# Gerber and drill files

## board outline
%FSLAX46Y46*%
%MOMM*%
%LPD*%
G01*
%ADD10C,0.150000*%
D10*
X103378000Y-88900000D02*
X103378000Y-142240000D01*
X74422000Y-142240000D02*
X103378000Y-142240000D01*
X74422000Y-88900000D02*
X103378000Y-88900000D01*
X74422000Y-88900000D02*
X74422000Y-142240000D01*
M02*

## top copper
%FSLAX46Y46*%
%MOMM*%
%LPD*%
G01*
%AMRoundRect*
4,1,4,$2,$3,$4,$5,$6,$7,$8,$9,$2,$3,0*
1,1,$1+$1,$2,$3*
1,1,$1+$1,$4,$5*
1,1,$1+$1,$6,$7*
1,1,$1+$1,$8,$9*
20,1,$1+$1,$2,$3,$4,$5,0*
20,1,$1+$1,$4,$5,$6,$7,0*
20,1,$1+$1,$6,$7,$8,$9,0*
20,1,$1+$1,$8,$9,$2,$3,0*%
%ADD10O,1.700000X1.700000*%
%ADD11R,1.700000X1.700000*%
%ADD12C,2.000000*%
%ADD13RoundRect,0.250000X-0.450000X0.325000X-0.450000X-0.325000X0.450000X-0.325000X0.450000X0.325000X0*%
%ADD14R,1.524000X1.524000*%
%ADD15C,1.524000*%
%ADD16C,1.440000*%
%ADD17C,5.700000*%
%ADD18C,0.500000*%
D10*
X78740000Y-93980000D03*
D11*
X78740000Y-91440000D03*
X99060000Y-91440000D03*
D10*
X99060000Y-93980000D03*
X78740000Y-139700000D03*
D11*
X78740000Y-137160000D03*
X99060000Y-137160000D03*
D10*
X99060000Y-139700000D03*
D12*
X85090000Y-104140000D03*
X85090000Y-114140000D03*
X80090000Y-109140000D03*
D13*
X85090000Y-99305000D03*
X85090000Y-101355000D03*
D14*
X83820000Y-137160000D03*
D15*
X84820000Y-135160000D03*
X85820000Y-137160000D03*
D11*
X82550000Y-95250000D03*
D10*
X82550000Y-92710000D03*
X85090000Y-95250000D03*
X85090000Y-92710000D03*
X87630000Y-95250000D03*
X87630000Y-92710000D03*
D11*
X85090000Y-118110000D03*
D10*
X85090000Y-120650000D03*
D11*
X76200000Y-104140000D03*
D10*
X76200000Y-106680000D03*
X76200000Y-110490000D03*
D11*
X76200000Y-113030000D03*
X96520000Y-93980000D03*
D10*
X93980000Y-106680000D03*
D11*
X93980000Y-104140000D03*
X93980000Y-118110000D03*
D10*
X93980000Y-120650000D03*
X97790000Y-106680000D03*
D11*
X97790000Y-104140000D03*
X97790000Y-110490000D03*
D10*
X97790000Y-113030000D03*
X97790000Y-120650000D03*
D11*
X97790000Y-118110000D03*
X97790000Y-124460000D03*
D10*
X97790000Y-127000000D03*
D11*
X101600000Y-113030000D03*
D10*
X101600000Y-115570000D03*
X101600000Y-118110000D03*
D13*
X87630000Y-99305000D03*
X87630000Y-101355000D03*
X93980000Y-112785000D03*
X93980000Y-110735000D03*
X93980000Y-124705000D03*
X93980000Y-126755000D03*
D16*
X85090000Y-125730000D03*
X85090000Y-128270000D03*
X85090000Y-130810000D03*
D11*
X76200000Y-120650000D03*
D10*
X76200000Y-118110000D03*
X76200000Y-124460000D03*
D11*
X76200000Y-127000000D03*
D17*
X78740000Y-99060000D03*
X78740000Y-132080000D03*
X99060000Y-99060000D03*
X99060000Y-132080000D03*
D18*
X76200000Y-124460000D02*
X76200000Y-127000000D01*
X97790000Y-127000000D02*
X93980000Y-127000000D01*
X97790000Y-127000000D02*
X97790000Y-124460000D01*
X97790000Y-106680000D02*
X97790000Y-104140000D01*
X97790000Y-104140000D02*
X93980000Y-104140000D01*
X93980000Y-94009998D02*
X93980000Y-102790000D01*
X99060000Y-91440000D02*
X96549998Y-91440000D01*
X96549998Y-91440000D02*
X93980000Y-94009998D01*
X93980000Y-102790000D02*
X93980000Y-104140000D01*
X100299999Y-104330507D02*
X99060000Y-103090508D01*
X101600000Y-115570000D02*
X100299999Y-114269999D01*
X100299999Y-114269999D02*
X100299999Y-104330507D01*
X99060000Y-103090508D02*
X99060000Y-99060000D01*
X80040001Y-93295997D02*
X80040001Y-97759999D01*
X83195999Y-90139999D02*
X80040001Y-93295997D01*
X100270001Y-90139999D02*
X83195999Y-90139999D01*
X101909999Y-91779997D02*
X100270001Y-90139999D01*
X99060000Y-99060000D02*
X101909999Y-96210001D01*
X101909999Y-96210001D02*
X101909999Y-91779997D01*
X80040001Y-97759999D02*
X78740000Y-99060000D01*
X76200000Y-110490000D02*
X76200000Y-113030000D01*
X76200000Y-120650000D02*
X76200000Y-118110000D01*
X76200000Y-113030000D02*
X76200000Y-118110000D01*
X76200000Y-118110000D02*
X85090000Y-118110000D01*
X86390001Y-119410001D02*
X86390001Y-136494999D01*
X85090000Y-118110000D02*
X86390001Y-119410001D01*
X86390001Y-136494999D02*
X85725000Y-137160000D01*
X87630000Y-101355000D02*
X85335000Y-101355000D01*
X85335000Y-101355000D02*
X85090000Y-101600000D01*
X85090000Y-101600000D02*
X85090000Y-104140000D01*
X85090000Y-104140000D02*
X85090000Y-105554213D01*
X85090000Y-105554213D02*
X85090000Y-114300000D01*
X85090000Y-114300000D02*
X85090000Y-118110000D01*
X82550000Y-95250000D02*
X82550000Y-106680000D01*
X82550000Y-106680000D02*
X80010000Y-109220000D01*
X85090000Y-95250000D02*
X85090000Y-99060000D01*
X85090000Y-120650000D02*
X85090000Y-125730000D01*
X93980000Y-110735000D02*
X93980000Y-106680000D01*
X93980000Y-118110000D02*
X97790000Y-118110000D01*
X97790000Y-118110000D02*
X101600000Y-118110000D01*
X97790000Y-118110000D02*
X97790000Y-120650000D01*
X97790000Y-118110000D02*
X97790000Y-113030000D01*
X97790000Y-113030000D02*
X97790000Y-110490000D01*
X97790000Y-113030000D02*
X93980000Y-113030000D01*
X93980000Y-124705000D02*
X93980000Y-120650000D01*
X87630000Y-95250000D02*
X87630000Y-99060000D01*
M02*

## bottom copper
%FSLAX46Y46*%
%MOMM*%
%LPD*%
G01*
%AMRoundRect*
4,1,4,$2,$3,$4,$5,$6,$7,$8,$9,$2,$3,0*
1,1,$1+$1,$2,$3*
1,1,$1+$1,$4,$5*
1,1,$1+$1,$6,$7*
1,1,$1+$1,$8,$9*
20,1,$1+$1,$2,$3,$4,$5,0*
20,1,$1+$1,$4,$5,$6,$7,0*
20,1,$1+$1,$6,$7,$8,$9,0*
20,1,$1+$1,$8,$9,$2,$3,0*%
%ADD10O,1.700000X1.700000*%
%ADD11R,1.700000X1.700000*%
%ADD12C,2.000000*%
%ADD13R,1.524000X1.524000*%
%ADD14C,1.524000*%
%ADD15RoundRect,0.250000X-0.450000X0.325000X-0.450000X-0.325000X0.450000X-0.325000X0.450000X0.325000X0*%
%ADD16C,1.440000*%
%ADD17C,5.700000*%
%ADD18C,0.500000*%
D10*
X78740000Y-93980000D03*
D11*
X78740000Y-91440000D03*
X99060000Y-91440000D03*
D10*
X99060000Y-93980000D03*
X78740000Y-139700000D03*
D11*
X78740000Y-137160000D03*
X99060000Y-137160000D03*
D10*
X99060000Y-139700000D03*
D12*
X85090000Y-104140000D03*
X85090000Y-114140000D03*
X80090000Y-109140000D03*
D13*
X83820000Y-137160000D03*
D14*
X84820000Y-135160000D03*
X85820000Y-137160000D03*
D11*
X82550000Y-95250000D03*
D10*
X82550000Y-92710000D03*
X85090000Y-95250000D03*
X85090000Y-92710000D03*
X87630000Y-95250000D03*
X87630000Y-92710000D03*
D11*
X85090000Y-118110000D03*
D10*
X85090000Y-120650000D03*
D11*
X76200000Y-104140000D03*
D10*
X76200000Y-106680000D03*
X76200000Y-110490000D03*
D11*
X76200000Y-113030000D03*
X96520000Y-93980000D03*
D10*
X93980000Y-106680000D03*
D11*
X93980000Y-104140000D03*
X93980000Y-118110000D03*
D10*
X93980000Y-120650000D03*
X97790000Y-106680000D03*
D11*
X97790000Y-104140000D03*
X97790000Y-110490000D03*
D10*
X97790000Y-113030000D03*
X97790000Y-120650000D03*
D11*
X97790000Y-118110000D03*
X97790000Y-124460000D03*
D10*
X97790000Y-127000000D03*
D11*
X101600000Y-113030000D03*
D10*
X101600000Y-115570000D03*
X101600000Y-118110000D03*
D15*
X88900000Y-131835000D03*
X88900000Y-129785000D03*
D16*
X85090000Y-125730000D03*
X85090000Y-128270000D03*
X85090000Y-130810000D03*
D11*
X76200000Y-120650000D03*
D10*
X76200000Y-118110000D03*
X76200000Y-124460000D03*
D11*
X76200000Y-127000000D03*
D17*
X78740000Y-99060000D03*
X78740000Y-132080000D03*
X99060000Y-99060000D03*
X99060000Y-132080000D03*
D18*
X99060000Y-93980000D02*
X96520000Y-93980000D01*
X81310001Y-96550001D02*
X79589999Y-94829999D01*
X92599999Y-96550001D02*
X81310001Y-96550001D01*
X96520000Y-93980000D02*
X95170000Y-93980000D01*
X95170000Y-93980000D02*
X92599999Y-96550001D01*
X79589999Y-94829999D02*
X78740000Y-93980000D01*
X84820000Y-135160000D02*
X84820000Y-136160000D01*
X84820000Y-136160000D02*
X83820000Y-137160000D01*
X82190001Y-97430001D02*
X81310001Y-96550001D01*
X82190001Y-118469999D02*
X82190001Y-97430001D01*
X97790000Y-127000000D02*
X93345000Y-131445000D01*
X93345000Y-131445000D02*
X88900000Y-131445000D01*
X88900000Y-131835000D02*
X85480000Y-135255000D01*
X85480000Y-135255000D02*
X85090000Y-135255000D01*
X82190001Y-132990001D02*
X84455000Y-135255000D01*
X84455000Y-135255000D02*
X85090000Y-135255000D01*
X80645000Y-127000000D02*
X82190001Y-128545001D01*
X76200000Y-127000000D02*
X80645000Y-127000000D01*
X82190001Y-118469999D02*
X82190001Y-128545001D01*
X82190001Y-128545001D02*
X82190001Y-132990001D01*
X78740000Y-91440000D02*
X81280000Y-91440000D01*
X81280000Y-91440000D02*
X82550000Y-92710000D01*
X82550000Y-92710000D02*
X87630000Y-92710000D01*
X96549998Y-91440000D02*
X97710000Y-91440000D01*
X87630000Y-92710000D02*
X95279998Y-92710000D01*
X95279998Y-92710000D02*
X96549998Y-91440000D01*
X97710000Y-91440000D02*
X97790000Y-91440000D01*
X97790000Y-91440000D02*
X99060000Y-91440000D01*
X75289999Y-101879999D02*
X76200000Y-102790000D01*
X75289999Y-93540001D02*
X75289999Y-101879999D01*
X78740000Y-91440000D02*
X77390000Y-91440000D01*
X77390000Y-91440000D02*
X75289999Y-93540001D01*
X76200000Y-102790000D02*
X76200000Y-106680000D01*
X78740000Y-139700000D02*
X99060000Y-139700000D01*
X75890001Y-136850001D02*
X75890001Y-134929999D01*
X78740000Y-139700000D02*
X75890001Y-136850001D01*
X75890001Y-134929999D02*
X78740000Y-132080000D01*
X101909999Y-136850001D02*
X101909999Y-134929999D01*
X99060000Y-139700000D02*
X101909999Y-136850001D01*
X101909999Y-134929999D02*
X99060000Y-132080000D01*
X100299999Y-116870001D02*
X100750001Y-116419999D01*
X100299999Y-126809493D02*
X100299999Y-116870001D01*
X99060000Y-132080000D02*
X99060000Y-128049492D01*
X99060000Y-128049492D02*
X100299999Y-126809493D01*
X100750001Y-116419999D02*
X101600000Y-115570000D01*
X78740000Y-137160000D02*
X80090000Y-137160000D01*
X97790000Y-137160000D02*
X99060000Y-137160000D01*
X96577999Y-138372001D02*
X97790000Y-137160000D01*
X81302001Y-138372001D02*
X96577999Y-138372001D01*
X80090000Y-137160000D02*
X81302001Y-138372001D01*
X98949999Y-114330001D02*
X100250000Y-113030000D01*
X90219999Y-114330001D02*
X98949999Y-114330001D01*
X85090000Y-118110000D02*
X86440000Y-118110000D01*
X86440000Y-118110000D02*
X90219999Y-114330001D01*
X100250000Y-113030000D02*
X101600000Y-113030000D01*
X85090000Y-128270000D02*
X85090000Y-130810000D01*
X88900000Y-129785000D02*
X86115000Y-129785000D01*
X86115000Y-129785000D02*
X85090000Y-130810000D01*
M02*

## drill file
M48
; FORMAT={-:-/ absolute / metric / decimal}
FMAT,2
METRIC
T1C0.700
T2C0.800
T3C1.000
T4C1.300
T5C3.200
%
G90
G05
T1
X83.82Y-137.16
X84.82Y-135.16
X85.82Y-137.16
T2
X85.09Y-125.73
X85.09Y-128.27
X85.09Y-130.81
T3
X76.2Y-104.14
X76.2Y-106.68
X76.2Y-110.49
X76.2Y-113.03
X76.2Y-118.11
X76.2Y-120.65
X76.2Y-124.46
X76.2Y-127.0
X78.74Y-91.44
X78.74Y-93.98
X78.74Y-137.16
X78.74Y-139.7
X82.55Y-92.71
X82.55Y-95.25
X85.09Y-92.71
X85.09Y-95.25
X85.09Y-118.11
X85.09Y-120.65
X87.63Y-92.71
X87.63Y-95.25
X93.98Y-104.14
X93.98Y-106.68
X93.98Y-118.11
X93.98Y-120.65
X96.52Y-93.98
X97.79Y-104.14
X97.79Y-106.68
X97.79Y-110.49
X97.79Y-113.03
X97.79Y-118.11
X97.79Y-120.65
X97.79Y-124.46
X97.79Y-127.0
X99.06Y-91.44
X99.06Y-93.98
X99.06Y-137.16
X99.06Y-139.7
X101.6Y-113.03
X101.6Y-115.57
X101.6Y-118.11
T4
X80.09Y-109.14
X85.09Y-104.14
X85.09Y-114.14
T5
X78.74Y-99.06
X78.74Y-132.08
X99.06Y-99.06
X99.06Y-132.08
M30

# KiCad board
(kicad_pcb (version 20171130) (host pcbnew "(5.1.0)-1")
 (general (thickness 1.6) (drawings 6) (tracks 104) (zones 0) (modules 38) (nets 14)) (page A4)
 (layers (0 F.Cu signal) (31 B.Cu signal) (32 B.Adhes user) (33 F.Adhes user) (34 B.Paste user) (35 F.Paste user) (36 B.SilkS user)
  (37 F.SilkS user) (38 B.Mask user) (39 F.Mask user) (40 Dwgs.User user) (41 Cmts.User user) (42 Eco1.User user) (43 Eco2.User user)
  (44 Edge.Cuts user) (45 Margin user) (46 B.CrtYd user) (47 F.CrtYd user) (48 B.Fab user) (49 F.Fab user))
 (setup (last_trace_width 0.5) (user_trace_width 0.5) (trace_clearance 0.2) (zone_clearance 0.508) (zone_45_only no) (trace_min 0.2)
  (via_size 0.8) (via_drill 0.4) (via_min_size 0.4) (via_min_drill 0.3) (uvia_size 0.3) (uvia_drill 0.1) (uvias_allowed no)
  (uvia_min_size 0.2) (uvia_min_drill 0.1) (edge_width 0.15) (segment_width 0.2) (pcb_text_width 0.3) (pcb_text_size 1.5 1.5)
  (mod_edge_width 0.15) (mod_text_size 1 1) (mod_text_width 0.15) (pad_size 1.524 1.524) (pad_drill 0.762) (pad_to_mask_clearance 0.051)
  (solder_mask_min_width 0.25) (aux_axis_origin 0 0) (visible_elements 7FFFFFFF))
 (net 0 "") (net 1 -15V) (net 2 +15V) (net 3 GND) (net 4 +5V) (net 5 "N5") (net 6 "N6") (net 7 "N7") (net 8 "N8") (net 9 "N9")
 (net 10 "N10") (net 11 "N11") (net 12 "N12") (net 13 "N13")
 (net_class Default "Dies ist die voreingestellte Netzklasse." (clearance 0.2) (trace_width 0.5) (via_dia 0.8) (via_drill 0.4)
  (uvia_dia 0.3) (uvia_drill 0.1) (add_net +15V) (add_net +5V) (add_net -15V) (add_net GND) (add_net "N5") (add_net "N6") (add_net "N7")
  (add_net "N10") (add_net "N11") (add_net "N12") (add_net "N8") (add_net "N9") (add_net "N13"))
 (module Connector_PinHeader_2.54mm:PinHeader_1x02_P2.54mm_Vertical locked (layer B.Cu) (at 78.74 91.44 180)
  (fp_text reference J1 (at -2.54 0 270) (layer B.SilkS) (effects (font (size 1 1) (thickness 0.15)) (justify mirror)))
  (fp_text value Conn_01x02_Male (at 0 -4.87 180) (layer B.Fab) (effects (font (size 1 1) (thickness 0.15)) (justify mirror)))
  (pad 2 thru_hole oval (at 0 -2.54 180) (size 1.7 1.7) (drill 1) (layers *.Cu *.Mask) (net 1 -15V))
  (pad 1 thru_hole rect (at 0 0 180) (size 1.7 1.7) (drill 1) (layers *.Cu *.Mask) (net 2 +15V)))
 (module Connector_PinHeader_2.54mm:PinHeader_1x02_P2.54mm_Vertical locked (layer B.Cu) (at 99.06 91.44 180)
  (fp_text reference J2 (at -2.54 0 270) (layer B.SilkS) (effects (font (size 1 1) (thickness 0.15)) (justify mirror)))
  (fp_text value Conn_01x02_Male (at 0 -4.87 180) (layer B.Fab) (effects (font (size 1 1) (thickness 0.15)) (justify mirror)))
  (pad 1 thru_hole rect (at 0 0 180) (size 1.7 1.7) (drill 1) (layers *.Cu *.Mask) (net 2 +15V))
  (pad 2 thru_hole oval (at 0 -2.54 180) (size 1.7 1.7) (drill 1) (layers *.Cu *.Mask) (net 1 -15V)))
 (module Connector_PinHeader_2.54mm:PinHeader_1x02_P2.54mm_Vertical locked (layer B.Cu) (at 78.74 137.16 180)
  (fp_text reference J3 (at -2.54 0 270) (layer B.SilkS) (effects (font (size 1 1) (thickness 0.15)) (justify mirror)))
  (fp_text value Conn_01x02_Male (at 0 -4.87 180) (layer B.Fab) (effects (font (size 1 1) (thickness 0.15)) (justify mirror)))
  (pad 2 thru_hole oval (at 0 -2.54 180) (size 1.7 1.7) (drill 1) (layers *.Cu *.Mask) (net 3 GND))
  (pad 1 thru_hole rect (at 0 0 180) (size 1.7 1.7) (drill 1) (layers *.Cu *.Mask) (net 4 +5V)))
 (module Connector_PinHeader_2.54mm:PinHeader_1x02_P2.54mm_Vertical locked (layer B.Cu) (at 99.06 137.16 180)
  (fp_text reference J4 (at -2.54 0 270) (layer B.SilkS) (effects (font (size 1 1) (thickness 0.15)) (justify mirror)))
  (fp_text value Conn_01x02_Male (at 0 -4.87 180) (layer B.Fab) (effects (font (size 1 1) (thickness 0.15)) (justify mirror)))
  (pad 1 thru_hole rect (at 0 0 180) (size 1.7 1.7) (drill 1) (layers *.Cu *.Mask) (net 4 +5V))
  (pad 2 thru_hole oval (at 0 -2.54 180) (size 1.7 1.7) (drill 1) (layers *.Cu *.Mask) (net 3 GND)))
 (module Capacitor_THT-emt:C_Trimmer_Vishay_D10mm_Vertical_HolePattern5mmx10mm (layer F.Cu) (at 85.09 104.14 270)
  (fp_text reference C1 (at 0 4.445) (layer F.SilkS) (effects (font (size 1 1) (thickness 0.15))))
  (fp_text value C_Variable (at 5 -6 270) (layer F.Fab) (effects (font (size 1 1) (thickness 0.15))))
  (pad 1 thru_hole circle (at 0 0 270) (size 2 2) (drill 1.3) (layers *.Cu *.Mask) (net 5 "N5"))
  (pad 1 thru_hole circle (at 10 0 270) (size 2 2) (drill 1.3) (layers *.Cu *.Mask) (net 5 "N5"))
  (pad 2 thru_hole circle (at 5 5 270) (size 2 2) (drill 1.3) (layers *.Cu *.Mask) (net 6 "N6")))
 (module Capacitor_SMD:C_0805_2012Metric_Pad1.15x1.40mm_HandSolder (layer F.Cu) (at 85.09 100.33 270)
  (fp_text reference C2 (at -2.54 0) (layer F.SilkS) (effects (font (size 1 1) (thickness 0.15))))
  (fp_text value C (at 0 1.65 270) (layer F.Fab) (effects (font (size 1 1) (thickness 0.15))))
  (pad 1 smd roundrect (at -1.025 0 270) (size 1.15 1.4) (layers F.Cu F.Paste F.Mask) (roundrect_rratio 0.217391) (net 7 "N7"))
  (pad 2 smd roundrect (at 1.025 0 270) (size 1.15 1.4) (layers F.Cu F.Paste F.Mask) (roundrect_rratio 0.217391) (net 5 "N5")))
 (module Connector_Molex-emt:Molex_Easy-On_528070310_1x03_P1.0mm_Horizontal (layer F.Cu) (at 83.82 137.16)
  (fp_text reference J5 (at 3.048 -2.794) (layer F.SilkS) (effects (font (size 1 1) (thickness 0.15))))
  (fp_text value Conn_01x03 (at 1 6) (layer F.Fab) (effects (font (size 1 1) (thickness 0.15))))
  (pad 1 thru_hole rect (at 0 0) (size 1.524 1.524) (drill 0.7) (layers *.Cu *.Mask) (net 1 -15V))
  (pad 2 thru_hole circle (at 1 -2) (size 1.524 1.524) (drill 0.7) (layers *.Cu *.Mask) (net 1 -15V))
  (pad 3 thru_hole circle (at 2 0) (size 1.524 1.524) (drill 0.7) (layers *.Cu *.Mask) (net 5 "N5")))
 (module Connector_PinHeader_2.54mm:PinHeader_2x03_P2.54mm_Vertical (layer F.Cu) (at 82.55 95.25 90)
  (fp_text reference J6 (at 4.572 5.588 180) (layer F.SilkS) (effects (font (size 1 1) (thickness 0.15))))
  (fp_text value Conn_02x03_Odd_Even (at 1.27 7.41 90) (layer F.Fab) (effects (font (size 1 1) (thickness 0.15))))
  (pad 1 thru_hole rect (at 0 0 90) (size 1.7 1.7) (drill 1) (layers *.Cu *.Mask) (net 6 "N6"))
  (pad 2 thru_hole oval (at 2.54 0 90) (size 1.7 1.7) (drill 1) (layers *.Cu *.Mask) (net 2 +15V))
  (pad 3 thru_hole oval (at 0 2.54 90) (size 1.7 1.7) (drill 1) (layers *.Cu *.Mask) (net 7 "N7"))
  (pad 4 thru_hole oval (at 2.54 2.54 90) (size 1.7 1.7) (drill 1) (layers *.Cu *.Mask) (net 2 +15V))
  (pad 5 thru_hole oval (at 0 5.08 90) (size 1.7 1.7) (drill 1) (layers *.Cu *.Mask) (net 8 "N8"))
  (pad 6 thru_hole oval (at 2.54 5.08 90) (size 1.7 1.7) (drill 1) (layers *.Cu *.Mask) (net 2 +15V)))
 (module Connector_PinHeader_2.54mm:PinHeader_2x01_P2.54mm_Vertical (layer F.Cu) (at 85.09 118.11 270)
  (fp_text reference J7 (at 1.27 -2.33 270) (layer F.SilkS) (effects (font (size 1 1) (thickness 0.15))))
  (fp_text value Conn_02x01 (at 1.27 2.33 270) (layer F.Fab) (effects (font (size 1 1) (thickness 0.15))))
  (pad 1 thru_hole rect (at 0 0 270) (size 1.7 1.7) (drill 1) (layers *.Cu *.Mask) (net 5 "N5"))
  (pad 2 thru_hole oval (at 2.54 0 270) (size 1.7 1.7) (drill 1) (layers *.Cu *.Mask) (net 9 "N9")))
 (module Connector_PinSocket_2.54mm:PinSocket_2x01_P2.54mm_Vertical (layer F.Cu) (at 76.2 104.14 90)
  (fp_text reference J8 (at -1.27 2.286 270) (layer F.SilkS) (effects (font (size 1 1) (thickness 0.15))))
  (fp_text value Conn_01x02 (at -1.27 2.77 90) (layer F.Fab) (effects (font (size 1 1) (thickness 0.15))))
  (pad 1 thru_hole rect (at 0 0 90) (size 1.7 1.7) (drill 1) (layers *.Cu *.Mask) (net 2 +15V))
  (pad 2 thru_hole oval (at -2.54 0 90) (size 1.7 1.7) (drill 1) (layers *.Cu *.Mask) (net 2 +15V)))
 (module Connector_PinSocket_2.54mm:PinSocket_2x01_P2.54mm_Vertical (layer F.Cu) (at 76.2 113.03 270)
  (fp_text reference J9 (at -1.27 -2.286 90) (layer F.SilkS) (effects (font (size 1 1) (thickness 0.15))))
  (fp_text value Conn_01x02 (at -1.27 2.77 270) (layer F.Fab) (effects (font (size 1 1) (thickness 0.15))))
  (pad 2 thru_hole oval (at -2.54 0 270) (size 1.7 1.7) (drill 1) (layers *.Cu *.Mask) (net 5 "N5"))
  (pad 1 thru_hole rect (at 0 0 270) (size 1.7 1.7) (drill 1) (layers *.Cu *.Mask) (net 5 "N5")))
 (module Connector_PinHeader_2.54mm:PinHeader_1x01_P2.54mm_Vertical (layer F.Cu) (at 96.52 93.98)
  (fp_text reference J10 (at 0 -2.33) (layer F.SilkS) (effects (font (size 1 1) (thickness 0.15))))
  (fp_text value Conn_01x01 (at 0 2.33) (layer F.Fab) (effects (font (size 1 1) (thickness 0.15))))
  (pad 1 thru_hole rect (at 0 0) (size 1.7 1.7) (drill 1) (layers *.Cu *.Mask) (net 1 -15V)))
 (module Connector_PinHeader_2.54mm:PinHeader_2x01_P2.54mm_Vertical (layer F.Cu) (at 93.98 104.14 270)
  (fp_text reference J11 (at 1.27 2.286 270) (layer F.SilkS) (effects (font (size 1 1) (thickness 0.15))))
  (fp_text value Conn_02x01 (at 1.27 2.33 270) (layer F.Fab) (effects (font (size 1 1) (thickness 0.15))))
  (pad 2 thru_hole oval (at 2.54 0 270) (size 1.7 1.7) (drill 1) (layers *.Cu *.Mask) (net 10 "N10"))
  (pad 1 thru_hole rect (at 0 0 270) (size 1.7 1.7) (drill 1) (layers *.Cu *.Mask) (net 2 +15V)))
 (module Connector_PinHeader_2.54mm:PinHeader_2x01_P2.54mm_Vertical (layer F.Cu) (at 93.98 118.11 270)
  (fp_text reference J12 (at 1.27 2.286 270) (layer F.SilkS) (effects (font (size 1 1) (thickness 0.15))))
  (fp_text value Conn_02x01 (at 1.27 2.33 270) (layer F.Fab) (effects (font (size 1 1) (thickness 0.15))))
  (pad 1 thru_hole rect (at 0 0 270) (size 1.7 1.7) (drill 1) (layers *.Cu *.Mask) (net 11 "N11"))
  (pad 2 thru_hole oval (at 2.54 0 270) (size 1.7 1.7) (drill 1) (layers *.Cu *.Mask) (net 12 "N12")))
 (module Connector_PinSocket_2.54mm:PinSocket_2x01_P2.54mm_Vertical (layer F.Cu) (at 97.79 104.14 90)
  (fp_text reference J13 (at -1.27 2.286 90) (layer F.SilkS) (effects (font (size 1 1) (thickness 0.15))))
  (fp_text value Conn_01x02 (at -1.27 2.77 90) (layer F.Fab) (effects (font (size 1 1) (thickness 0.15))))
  (pad 2 thru_hole oval (at -2.54 0 90) (size 1.7 1.7) (drill 1) (layers *.Cu *.Mask) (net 2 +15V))
  (pad 1 thru_hole rect (at 0 0 90) (size 1.7 1.7) (drill 1) (layers *.Cu *.Mask) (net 2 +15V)))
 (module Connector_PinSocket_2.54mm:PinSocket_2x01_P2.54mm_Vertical (layer F.Cu) (at 97.79 110.49 90)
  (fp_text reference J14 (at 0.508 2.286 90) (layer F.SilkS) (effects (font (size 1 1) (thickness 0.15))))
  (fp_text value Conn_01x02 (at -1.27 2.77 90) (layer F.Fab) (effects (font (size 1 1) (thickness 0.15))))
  (pad 1 thru_hole rect (at 0 0 90) (size 1.7 1.7) (drill 1) (layers *.Cu *.Mask) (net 11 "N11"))
  (pad 2 thru_hole oval (at -2.54 0 90) (size 1.7 1.7) (drill 1) (layers *.Cu *.Mask) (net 11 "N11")))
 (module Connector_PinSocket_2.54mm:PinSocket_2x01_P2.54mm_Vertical (layer F.Cu) (at 97.79 118.11 90)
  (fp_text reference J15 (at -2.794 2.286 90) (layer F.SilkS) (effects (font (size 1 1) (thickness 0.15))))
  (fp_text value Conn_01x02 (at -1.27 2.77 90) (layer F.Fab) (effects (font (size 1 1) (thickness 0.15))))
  (pad 2 thru_hole oval (at -2.54 0 90) (size 1.7 1.7) (drill 1) (layers *.Cu *.Mask) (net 11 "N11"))
  (pad 1 thru_hole rect (at 0 0 90) (size 1.7 1.7) (drill 1) (layers *.Cu *.Mask) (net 11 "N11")))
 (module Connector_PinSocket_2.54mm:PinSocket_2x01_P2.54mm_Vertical (layer F.Cu) (at 97.79 124.46 90)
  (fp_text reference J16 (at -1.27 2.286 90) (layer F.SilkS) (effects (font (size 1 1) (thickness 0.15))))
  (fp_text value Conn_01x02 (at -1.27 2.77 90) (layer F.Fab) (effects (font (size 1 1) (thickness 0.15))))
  (pad 1 thru_hole rect (at 0 0 90) (size 1.7 1.7) (drill 1) (layers *.Cu *.Mask) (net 1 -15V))
  (pad 2 thru_hole oval (at -2.54 0 90) (size 1.7 1.7) (drill 1) (layers *.Cu *.Mask) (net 1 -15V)))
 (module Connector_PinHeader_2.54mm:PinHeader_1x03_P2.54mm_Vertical (layer F.Cu) (at 101.6 113.03)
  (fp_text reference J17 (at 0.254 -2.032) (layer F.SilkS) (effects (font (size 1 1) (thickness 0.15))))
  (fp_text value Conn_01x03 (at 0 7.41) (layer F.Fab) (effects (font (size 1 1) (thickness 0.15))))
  (pad 1 thru_hole rect (at 0 0) (size 1.7 1.7) (drill 1) (layers *.Cu *.Mask) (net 5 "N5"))
  (pad 2 thru_hole oval (at 0 2.54) (size 1.7 1.7) (drill 1) (layers *.Cu *.Mask) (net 3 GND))
  (pad 3 thru_hole oval (at 0 5.08) (size 1.7 1.7) (drill 1) (layers *.Cu *.Mask) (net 11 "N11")))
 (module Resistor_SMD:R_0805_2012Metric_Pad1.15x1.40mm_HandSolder (layer F.Cu) (at 87.63 100.33 270)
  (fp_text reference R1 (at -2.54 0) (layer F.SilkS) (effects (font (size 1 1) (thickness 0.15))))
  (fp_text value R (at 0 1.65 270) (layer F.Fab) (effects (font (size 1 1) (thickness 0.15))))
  (pad 1 smd roundrect (at -1.025 0 270) (size 1.15 1.4) (layers F.Cu F.Paste F.Mask) (roundrect_rratio 0.217391) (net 8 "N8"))
  (pad 2 smd roundrect (at 1.025 0 270) (size 1.15 1.4) (layers F.Cu F.Paste F.Mask) (roundrect_rratio 0.217391) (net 5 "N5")))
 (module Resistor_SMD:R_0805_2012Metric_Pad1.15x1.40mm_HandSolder (layer B.Cu) (at 88.9 130.81 270)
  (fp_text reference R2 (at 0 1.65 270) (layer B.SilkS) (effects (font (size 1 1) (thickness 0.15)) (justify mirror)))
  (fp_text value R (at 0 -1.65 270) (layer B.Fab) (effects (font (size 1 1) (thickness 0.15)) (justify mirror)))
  (pad 2 smd roundrect (at 1.025 0 270) (size 1.15 1.4) (layers B.Cu B.Paste B.Mask) (roundrect_rratio 0.217391) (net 1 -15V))
  (pad 1 smd roundrect (at -1.025 0 270) (size 1.15 1.4) (layers B.Cu B.Paste B.Mask) (roundrect_rratio 0.217391) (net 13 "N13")))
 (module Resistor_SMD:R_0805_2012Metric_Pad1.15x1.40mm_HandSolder (layer F.Cu) (at 93.98 111.76 270)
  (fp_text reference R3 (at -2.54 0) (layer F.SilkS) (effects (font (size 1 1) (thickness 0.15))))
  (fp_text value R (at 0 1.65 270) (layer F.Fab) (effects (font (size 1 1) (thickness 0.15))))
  (pad 2 smd roundrect (at 1.025 0 270) (size 1.15 1.4) (layers F.Cu F.Paste F.Mask) (roundrect_rratio 0.217391) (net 11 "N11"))
  (pad 1 smd roundrect (at -1.025 0 270) (size 1.15 1.4) (layers F.Cu F.Paste F.Mask) (roundrect_rratio 0.217391) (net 10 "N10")))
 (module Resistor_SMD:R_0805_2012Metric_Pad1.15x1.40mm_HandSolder (layer F.Cu) (at 93.98 125.73 270)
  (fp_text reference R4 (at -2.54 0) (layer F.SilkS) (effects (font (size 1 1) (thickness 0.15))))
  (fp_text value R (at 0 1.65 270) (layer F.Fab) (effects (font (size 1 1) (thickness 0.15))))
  (pad 1 smd roundrect (at -1.025 0 270) (size 1.15 1.4) (layers F.Cu F.Paste F.Mask) (roundrect_rratio 0.217391) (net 12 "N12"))
  (pad 2 smd roundrect (at 1.025 0 270) (size 1.15 1.4) (layers F.Cu F.Paste F.Mask) (roundrect_rratio 0.217391) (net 1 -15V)))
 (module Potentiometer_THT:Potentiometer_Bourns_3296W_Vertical (layer F.Cu) (at 85.09 125.73 90)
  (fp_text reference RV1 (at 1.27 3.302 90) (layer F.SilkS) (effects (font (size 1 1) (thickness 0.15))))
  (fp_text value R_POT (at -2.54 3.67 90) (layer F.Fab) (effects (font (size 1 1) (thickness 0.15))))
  (pad 1 thru_hole circle (at 0 0 90) (size 1.44 1.44) (drill 0.8) (layers *.Cu *.Mask) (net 9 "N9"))
  (pad 2 thru_hole circle (at -2.54 0 90) (size 1.44 1.44) (drill 0.8) (layers *.Cu *.Mask) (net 13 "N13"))
  (pad 3 thru_hole circle (at -5.08 0 90) (size 1.44 1.44) (drill 0.8) (layers *.Cu *.Mask) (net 13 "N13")))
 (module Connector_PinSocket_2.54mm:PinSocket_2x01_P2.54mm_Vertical (layer F.Cu) (at 76.2 120.65 270)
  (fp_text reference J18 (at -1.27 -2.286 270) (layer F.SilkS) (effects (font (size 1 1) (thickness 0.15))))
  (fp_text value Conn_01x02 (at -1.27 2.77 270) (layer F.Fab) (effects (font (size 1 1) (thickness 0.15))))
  (pad 1 thru_hole rect (at 0 0 270) (size 1.7 1.7) (drill 1) (layers *.Cu *.Mask) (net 5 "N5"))
  (pad 2 thru_hole oval (at -2.54 0 270) (size 1.7 1.7) (drill 1) (layers *.Cu *.Mask) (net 5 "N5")))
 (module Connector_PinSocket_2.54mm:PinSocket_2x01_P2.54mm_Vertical (layer F.Cu) (at 76.2 127 270)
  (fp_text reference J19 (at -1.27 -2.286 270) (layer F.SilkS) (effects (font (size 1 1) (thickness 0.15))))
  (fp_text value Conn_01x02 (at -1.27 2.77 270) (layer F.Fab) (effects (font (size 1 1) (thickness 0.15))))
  (pad 2 thru_hole oval (at -2.54 0 270) (size 1.7 1.7) (drill 1) (layers *.Cu *.Mask) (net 1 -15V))
  (pad 1 thru_hole rect (at 0 0 270) (size 1.7 1.7) (drill 1) (layers *.Cu *.Mask) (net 1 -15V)))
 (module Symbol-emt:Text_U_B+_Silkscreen (layer F.Cu) (at 75.184 91.44)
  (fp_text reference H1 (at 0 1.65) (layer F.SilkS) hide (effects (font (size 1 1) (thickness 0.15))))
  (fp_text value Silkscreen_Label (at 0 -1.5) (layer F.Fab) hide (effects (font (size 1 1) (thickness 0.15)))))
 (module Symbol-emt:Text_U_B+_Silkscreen (layer F.Cu) (at 101.092 91.44)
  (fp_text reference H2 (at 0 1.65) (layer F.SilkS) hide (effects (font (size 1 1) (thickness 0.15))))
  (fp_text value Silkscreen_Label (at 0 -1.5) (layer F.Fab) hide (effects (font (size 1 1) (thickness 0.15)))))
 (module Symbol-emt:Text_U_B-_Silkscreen (layer F.Cu) (at 75.184 93.98)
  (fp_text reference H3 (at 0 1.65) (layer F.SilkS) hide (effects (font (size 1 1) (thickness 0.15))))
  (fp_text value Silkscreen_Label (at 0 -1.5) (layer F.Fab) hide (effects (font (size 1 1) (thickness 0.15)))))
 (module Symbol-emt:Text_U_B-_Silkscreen (layer F.Cu) (at 101.092 93.98)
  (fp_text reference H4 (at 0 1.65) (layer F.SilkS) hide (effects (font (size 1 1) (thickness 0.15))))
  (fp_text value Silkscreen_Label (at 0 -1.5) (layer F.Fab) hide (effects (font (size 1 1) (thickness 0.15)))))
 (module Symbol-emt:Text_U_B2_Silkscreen (layer F.Cu) (at 75.184 137.16)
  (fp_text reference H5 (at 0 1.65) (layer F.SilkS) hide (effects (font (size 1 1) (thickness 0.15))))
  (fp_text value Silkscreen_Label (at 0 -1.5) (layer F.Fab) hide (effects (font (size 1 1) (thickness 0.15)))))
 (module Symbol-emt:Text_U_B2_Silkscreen (layer F.Cu) (at 101.092 137.16)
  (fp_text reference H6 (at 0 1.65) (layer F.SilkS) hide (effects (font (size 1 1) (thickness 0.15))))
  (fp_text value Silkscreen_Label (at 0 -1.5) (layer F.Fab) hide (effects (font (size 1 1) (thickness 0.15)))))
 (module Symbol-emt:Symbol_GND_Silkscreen (layer F.Cu) (at 75.692 139.7)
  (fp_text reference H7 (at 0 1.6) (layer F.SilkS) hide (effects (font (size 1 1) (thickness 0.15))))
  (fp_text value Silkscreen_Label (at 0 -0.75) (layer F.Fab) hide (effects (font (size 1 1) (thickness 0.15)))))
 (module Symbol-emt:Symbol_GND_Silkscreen (layer F.Cu) (at 102.108 139.7)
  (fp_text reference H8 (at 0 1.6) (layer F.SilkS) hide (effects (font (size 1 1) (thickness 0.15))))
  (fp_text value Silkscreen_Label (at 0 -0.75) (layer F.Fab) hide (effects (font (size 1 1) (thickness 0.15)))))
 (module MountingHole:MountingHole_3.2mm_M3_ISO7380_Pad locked (layer F.Cu) (at 78.74 99.06)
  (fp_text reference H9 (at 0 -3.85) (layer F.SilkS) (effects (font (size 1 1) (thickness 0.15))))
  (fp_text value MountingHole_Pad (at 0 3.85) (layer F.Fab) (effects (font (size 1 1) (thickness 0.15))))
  (pad 1 thru_hole circle (at 0 0) (size 5.7 5.7) (drill 3.2) (layers *.Cu *.Mask) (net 3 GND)))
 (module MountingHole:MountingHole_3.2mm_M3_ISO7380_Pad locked (layer F.Cu) (at 78.74 132.08)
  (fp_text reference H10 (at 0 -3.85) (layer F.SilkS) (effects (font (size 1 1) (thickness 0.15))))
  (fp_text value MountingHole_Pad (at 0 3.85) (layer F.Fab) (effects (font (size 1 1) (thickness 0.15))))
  (pad 1 thru_hole circle (at 0 0) (size 5.7 5.7) (drill 3.2) (layers *.Cu *.Mask) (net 3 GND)))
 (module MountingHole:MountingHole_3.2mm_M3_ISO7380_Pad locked (layer F.Cu) (at 99.06 99.06)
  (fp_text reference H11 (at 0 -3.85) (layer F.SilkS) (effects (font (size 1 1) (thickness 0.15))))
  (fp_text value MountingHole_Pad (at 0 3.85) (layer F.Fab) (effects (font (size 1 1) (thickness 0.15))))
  (pad 1 thru_hole circle (at 0 0) (size 5.7 5.7) (drill 3.2) (layers *.Cu *.Mask) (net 3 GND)))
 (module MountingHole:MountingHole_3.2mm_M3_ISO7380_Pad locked (layer F.Cu) (at 99.06 132.08)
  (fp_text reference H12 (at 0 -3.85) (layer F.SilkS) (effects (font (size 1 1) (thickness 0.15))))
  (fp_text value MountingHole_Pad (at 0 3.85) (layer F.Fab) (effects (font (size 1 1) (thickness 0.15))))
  (pad 1 thru_hole circle (at 0 0) (size 5.7 5.7) (drill 3.2) (layers *.Cu *.Mask) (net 3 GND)))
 (gr_line (start 103.378 88.9) (end 103.378 142.24) (layer Edge.Cuts) (width 0.15))
 (gr_line (start 74.422 142.24) (end 103.378 142.24) (layer Edge.Cuts) (width 0.15))
 (gr_line (start 74.422 88.9) (end 103.378 88.9) (layer Edge.Cuts) (width 0.15))
 (gr_line (start 74.422 88.9) (end 74.422 142.24) (layer Edge.Cuts) (width 0.15))
 (segment (start 76.2 124.46) (end 76.2 127) (width 0.5) (layer F.Cu) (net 1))
 (segment (start 99.06 93.98) (end 96.52 93.98) (width 0.5) (layer B.Cu) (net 1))
 (segment (start 81.310001 96.550001) (end 79.589999 94.829999) (width 0.5) (layer B.Cu) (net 1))
 (segment (start 92.599999 96.550001) (end 81.310001 96.550001) (width 0.5) (layer B.Cu) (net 1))
 (segment (start 96.52 93.98) (end 95.17 93.98) (width 0.5) (layer B.Cu) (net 1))
 (segment (start 95.17 93.98) (end 92.599999 96.550001) (width 0.5) (layer B.Cu) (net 1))
 (segment (start 79.589999 94.829999) (end 78.74 93.98) (width 0.5) (layer B.Cu) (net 1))
 (segment (start 84.82 135.16) (end 84.82 136.16) (width 0.5) (layer B.Cu) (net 1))
 (segment (start 84.82 136.16) (end 83.82 137.16) (width 0.5) (layer B.Cu) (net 1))
 (segment (start 97.79 127) (end 93.98 127) (width 0.5) (layer F.Cu) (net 1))
 (segment (start 97.79 127) (end 97.79 124.46) (width 0.5) (layer F.Cu) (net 1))
 (segment (start 82.190001 97.430001) (end 81.310001 96.550001) (width 0.5) (layer B.Cu) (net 1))
 (segment (start 82.190001 118.469999) (end 82.190001 97.430001) (width 0.5) (layer B.Cu) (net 1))
 (segment (start 97.79 127) (end 93.345 131.445) (width 0.5) (layer B.Cu) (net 1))
 (segment (start 93.345 131.445) (end 88.9 131.445) (width 0.5) (layer B.Cu) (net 1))
 (segment (start 88.9 131.835) (end 85.48 135.255) (width 0.5) (layer B.Cu) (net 1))
 (segment (start 85.48 135.255) (end 85.09 135.255) (width 0.5) (layer B.Cu) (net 1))
 (segment (start 82.190001 132.990001) (end 84.455 135.255) (width 0.5) (layer B.Cu) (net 1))
 (segment (start 84.455 135.255) (end 85.09 135.255) (width 0.5) (layer B.Cu) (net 1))
 (segment (start 80.645 127) (end 82.190001 128.545001) (width 0.5) (layer B.Cu) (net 1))
 (segment (start 76.2 127) (end 80.645 127) (width 0.5) (layer B.Cu) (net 1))
 (segment (start 82.190001 118.469999) (end 82.190001 128.545001) (width 0.5) (layer B.Cu) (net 1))
 (segment (start 82.190001 128.545001) (end 82.190001 132.990001) (width 0.5) (layer B.Cu) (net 1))
 (segment (start 78.74 91.44) (end 81.28 91.44) (width 0.5) (layer B.Cu) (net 2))
 (segment (start 81.28 91.44) (end 82.55 92.71) (width 0.5) (layer B.Cu) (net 2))
 (segment (start 82.55 92.71) (end 87.63 92.71) (width 0.5) (layer B.Cu) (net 2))
 (segment (start 96.549998 91.44) (end 97.71 91.44) (width 0.5) (layer B.Cu) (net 2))
 (segment (start 87.63 92.71) (end 95.279998 92.71) (width 0.5) (layer B.Cu) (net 2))
 (segment (start 95.279998 92.71) (end 96.549998 91.44) (width 0.5) (layer B.Cu) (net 2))
 (segment (start 97.71 91.44) (end 97.79 91.44) (width 0.5) (layer B.Cu) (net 2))
 (segment (start 97.79 91.44) (end 99.06 91.44) (width 0.5) (layer B.Cu) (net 2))
 (segment (start 75.289999 101.879999) (end 76.2 102.79) (width 0.5) (layer B.Cu) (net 2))
 (segment (start 75.289999 93.540001) (end 75.289999 101.879999) (width 0.5) (layer B.Cu) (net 2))
 (segment (start 78.74 91.44) (end 77.39 91.44) (width 0.5) (layer B.Cu) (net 2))
 (segment (start 77.39 91.44) (end 75.289999 93.540001) (width 0.5) (layer B.Cu) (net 2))
 (segment (start 76.2 102.79) (end 76.2 106.68) (width 0.5) (layer B.Cu) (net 2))
 (segment (start 97.79 106.68) (end 97.79 104.14) (width 0.5) (layer F.Cu) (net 2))
 (segment (start 97.79 104.14) (end 93.98 104.14) (width 0.5) (layer F.Cu) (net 2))
 (segment (start 93.98 94.009998) (end 93.98 102.79) (width 0.5) (layer F.Cu) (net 2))
 (segment (start 99.06 91.44) (end 96.549998 91.44) (width 0.5) (layer F.Cu) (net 2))
 (segment (start 96.549998 91.44) (end 93.98 94.009998) (width 0.5) (layer F.Cu) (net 2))
 (segment (start 93.98 102.79) (end 93.98 104.14) (width 0.5) (layer F.Cu) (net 2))
 (segment (start 78.74 139.7) (end 99.06 139.7) (width 0.5) (layer B.Cu) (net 3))
 (segment (start 75.890001 136.850001) (end 75.890001 134.929999) (width 0.5) (layer B.Cu) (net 3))
 (segment (start 78.74 139.7) (end 75.890001 136.850001) (width 0.5) (layer B.Cu) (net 3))
 (segment (start 75.890001 134.929999) (end 78.74 132.08) (width 0.5) (layer B.Cu) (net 3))
 (segment (start 101.909999 136.850001) (end 101.909999 134.929999) (width 0.5) (layer B.Cu) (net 3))
 (segment (start 99.06 139.7) (end 101.909999 136.850001) (width 0.5) (layer B.Cu) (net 3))
 (segment (start 101.909999 134.929999) (end 99.06 132.08) (width 0.5) (layer B.Cu) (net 3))
 (segment (start 100.299999 116.870001) (end 100.750001 116.419999) (width 0.5) (layer B.Cu) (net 3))
 (segment (start 100.299999 126.809493) (end 100.299999 116.870001) (width 0.5) (layer B.Cu) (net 3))
 (segment (start 99.06 132.08) (end 99.06 128.049492) (width 0.5) (layer B.Cu) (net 3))
 (segment (start 99.06 128.049492) (end 100.299999 126.809493) (width 0.5) (layer B.Cu) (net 3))
 (segment (start 100.750001 116.419999) (end 101.6 115.57) (width 0.5) (layer B.Cu) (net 3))
 (segment (start 100.299999 104.330507) (end 99.06 103.090508) (width 0.5) (layer F.Cu) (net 3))
 (segment (start 101.6 115.57) (end 100.299999 114.269999) (width 0.5) (layer F.Cu) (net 3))
 (segment (start 100.299999 114.269999) (end 100.299999 104.330507) (width 0.5) (layer F.Cu) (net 3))
 (segment (start 99.06 103.090508) (end 99.06 99.06) (width 0.5) (layer F.Cu) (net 3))
 (segment (start 80.040001 93.295997) (end 80.040001 97.759999) (width 0.5) (layer F.Cu) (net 3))
 (segment (start 83.195999 90.139999) (end 80.040001 93.295997) (width 0.5) (layer F.Cu) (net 3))
 (segment (start 100.270001 90.139999) (end 83.195999 90.139999) (width 0.5) (layer F.Cu) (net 3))
 (segment (start 101.909999 91.779997) (end 100.270001 90.139999) (width 0.5) (layer F.Cu) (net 3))
 (segment (start 99.06 99.06) (end 101.909999 96.210001) (width 0.5) (layer F.Cu) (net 3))
 (segment (start 101.909999 96.210001) (end 101.909999 91.779997) (width 0.5) (layer F.Cu) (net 3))
 (segment (start 80.040001 97.759999) (end 78.74 99.06) (width 0.5) (layer F.Cu) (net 3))
 (segment (start 78.74 137.16) (end 80.09 137.16) (width 0.5) (layer B.Cu) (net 4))
 (segment (start 97.79 137.16) (end 99.06 137.16) (width 0.5) (layer B.Cu) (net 4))
 (segment (start 96.577999 138.372001) (end 97.79 137.16) (width 0.5) (layer B.Cu) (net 4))
 (segment (start 81.302001 138.372001) (end 96.577999 138.372001) (width 0.5) (layer B.Cu) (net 4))
 (segment (start 80.09 137.16) (end 81.302001 138.372001) (width 0.5) (layer B.Cu) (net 4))
 (segment (start 76.2 110.49) (end 76.2 113.03) (width 0.5) (layer F.Cu) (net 5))
 (segment (start 76.2 120.65) (end 76.2 118.11) (width 0.5) (layer F.Cu) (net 5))
 (segment (start 76.2 113.03) (end 76.2 118.11) (width 0.5) (layer F.Cu) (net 5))
 (segment (start 76.2 118.11) (end 85.09 118.11) (width 0.5) (layer F.Cu) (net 5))
 (segment (start 98.949999 114.330001) (end 100.25 113.03) (width 0.5) (layer B.Cu) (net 5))
 (segment (start 90.219999 114.330001) (end 98.949999 114.330001) (width 0.5) (layer B.Cu) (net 5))
 (segment (start 85.09 118.11) (end 86.44 118.11) (width 0.5) (layer B.Cu) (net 5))
 (segment (start 86.44 118.11) (end 90.219999 114.330001) (width 0.5) (layer B.Cu) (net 5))
 (segment (start 100.25 113.03) (end 101.6 113.03) (width 0.5) (layer B.Cu) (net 5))
 (segment (start 86.390001 119.410001) (end 86.390001 136.494999) (width 0.5) (layer F.Cu) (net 5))
 (segment (start 85.09 118.11) (end 86.390001 119.410001) (width 0.5) (layer F.Cu) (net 5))
 (segment (start 86.390001 136.494999) (end 85.725 137.16) (width 0.5) (layer F.Cu) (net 5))
 (segment (start 87.63 101.355) (end 85.335 101.355) (width 0.5) (layer F.Cu) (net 5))
 (segment (start 85.335 101.355) (end 85.09 101.6) (width 0.5) (layer F.Cu) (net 5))
 (segment (start 85.09 101.6) (end 85.09 104.14) (width 0.5) (layer F.Cu) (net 5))
 (segment (start 85.09 104.14) (end 85.09 105.554213) (width 0.5) (layer F.Cu) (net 5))
 (segment (start 85.09 105.554213) (end 85.09 114.3) (width 0.5) (layer F.Cu) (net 5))
 (segment (start 85.09 114.3) (end 85.09 118.11) (width 0.5) (layer F.Cu) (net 5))
 (segment (start 82.55 95.25) (end 82.55 106.68) (width 0.5) (layer F.Cu) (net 6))
 (segment (start 82.55 106.68) (end 80.01 109.22) (width 0.5) (layer F.Cu) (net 6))
 (segment (start 85.09 95.25) (end 85.09 99.06) (width 0.5) (layer F.Cu) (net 7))
 (segment (start 85.09 120.65) (end 85.09 125.73) (width 0.5) (layer F.Cu) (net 9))
 (segment (start 93.98 110.735) (end 93.98 106.68) (width 0.5) (layer F.Cu) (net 10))
 (segment (start 93.98 118.11) (end 97.79 118.11) (width 0.5) (layer F.Cu) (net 11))
 (segment (start 97.79 118.11) (end 101.6 118.11) (width 0.5) (layer F.Cu) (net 11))
 (segment (start 97.79 118.11) (end 97.79 120.65) (width 0.5) (layer F.Cu) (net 11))
 (segment (start 97.79 118.11) (end 97.79 113.03) (width 0.5) (layer F.Cu) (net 11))
 (segment (start 97.79 113.03) (end 97.79 110.49) (width 0.5) (layer F.Cu) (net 11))
 (segment (start 97.79 113.03) (end 93.98 113.03) (width 0.5) (layer F.Cu) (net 11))
 (segment (start 93.98 124.705) (end 93.98 120.65) (width 0.5) (layer F.Cu) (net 12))
 (segment (start 85.09 128.27) (end 85.09 130.81) (width 0.5) (layer B.Cu) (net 13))
 (segment (start 88.9 129.785) (end 86.115 129.785) (width 0.5) (layer B.Cu) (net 13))
 (segment (start 86.115 129.785) (end 85.09 130.81) (width 0.5) (layer B.Cu) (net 13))
 (segment (start 87.63 95.25) (end 87.63 99.06) (width 0.5) (layer F.Cu) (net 8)))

